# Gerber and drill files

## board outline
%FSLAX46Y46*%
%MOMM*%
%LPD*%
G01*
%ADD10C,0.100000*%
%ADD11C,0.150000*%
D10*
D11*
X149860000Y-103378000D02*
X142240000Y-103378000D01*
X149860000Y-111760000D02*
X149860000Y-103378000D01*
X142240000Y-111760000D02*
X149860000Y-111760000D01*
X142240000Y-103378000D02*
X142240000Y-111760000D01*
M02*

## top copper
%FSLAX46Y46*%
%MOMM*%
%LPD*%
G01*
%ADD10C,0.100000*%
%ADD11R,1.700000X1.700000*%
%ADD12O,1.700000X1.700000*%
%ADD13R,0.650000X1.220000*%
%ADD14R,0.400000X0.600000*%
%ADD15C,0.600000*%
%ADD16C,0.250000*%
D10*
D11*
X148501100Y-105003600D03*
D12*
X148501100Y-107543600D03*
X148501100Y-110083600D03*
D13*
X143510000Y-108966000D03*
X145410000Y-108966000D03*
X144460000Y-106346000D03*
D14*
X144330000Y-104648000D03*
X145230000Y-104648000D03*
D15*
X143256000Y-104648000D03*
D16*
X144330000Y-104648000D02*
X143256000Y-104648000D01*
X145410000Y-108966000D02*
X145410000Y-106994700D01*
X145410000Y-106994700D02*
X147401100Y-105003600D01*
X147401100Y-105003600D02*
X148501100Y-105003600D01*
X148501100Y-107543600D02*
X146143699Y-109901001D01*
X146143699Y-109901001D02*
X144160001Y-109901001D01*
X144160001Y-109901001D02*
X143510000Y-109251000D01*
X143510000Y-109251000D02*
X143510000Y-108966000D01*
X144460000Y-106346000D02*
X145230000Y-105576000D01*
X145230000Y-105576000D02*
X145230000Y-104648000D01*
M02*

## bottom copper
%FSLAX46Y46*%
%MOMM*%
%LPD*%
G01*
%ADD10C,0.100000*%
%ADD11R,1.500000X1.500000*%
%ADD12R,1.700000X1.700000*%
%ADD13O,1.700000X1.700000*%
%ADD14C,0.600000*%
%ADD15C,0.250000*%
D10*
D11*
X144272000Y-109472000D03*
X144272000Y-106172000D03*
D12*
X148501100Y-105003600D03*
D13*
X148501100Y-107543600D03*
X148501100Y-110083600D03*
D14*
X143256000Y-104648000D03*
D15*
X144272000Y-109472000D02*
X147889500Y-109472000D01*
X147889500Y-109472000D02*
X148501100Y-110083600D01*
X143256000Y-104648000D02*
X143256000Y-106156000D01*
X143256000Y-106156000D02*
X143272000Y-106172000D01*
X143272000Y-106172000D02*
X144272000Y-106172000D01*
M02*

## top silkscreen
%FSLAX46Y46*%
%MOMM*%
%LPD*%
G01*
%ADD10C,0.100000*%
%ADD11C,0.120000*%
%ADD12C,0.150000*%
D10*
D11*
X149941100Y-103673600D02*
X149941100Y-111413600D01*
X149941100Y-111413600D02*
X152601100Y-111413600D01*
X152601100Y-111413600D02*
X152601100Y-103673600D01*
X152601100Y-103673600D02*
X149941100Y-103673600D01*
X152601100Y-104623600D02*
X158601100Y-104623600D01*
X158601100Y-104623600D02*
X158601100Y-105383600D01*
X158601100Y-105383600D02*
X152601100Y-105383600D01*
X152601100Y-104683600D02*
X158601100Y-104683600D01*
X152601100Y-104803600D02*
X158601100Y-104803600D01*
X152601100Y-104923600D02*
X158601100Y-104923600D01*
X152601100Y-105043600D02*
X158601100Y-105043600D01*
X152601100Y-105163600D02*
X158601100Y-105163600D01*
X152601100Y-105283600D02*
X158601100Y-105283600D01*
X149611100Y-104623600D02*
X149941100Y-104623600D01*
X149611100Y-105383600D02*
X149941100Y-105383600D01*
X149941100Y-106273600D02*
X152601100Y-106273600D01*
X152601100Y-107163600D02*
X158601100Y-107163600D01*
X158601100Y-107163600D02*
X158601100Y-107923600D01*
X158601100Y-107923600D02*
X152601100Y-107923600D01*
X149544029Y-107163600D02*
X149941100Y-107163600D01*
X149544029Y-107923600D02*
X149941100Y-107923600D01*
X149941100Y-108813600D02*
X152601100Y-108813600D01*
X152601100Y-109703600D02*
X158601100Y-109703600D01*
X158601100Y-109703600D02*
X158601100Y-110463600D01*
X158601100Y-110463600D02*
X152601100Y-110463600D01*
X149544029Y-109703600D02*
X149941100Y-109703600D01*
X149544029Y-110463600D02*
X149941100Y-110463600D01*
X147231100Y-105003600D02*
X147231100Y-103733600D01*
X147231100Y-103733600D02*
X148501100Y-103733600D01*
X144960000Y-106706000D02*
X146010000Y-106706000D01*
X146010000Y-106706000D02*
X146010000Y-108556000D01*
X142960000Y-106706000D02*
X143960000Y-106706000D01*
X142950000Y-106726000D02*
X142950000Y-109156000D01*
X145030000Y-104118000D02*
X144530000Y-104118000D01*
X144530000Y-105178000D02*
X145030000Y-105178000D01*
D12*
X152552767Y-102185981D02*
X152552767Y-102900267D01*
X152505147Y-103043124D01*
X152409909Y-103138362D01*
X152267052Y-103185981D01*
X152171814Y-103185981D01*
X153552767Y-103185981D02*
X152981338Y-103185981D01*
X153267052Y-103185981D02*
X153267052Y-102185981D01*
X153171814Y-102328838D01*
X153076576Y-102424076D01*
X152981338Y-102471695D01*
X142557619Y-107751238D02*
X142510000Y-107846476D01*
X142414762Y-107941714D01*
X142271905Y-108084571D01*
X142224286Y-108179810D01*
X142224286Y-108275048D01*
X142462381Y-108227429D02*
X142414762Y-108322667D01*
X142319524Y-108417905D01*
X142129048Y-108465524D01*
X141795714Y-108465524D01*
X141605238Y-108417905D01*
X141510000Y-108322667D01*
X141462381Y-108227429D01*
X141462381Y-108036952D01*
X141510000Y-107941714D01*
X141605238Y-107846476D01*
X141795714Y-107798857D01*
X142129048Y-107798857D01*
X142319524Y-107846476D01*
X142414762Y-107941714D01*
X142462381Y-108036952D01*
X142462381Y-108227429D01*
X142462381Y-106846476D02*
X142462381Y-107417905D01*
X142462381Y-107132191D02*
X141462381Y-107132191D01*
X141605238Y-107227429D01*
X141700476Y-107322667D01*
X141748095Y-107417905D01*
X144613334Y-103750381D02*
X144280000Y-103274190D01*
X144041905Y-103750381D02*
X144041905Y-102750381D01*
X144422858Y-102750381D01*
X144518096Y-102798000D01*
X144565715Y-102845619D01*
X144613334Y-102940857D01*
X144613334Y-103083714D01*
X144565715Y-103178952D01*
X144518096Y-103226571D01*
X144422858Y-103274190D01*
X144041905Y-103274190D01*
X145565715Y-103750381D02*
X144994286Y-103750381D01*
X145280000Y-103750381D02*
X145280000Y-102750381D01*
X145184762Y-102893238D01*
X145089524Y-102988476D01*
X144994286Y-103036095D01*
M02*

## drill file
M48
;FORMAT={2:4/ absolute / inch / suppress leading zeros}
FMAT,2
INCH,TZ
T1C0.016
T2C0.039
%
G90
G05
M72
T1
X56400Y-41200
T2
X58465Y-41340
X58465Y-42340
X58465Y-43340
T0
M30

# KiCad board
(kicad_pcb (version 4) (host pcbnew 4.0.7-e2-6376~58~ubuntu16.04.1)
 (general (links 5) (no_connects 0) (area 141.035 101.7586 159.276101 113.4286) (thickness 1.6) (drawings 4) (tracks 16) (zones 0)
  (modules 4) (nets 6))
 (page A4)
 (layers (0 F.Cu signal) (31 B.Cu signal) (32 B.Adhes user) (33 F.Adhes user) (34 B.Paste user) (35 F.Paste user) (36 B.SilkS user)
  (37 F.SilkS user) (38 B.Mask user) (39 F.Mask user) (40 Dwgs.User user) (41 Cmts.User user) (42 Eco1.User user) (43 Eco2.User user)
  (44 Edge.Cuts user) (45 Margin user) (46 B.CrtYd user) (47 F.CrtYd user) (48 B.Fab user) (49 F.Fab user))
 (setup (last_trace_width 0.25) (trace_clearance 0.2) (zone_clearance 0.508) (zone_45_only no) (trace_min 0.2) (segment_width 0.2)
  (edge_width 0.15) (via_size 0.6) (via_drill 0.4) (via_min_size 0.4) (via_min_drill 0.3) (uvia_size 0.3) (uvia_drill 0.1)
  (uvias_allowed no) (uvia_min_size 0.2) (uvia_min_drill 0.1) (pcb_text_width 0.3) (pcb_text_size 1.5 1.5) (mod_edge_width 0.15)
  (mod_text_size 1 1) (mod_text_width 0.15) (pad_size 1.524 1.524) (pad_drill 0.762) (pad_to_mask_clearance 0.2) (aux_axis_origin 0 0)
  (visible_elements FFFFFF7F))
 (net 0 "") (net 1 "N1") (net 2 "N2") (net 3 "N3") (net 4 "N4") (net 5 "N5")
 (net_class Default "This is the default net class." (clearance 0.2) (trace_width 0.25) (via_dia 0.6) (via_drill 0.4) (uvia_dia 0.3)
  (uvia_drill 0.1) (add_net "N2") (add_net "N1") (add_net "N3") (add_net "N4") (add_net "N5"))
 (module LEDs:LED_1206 (layer B.Cu) (at 144.272 107.822 270)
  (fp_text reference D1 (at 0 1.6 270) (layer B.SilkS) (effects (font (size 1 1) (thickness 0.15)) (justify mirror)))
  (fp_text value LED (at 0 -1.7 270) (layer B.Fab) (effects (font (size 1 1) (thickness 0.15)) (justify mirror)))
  (pad 2 smd rect (at 1.65 0 90) (size 1.5 1.5) (layers B.Cu B.Paste B.Mask) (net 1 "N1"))
  (pad 1 smd rect (at -1.65 0 90) (size 1.5 1.5) (layers B.Cu B.Paste B.Mask) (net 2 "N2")))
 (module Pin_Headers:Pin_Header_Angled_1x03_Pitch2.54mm (layer F.Cu) (at 148.5011 105.0036)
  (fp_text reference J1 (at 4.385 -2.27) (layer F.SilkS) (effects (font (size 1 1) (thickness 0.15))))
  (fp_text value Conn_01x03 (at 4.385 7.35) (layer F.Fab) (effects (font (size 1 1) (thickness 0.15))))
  (fp_line (start 1.44 -1.33) (end 1.44 6.41) (layer F.SilkS) (width 0.12))
  (fp_line (start 1.44 6.41) (end 4.1 6.41) (layer F.SilkS) (width 0.12))
  (fp_line (start 4.1 6.41) (end 4.1 -1.33) (layer F.SilkS) (width 0.12))
  (fp_line (start 4.1 -1.33) (end 1.44 -1.33) (layer F.SilkS) (width 0.12))
  (fp_line (start 4.1 -0.38) (end 10.1 -0.38) (layer F.SilkS) (width 0.12))
  (fp_line (start 10.1 -0.38) (end 10.1 0.38) (layer F.SilkS) (width 0.12))
  (fp_line (start 10.1 0.38) (end 4.1 0.38) (layer F.SilkS) (width 0.12))
  (fp_line (start 4.1 -0.32) (end 10.1 -0.32) (layer F.SilkS) (width 0.12))
  (fp_line (start 4.1 -0.2) (end 10.1 -0.2) (layer F.SilkS) (width 0.12))
  (fp_line (start 4.1 -0.08) (end 10.1 -0.08) (layer F.SilkS) (width 0.12))
  (fp_line (start 4.1 0.04) (end 10.1 0.04) (layer F.SilkS) (width 0.12))
  (fp_line (start 4.1 0.16) (end 10.1 0.16) (layer F.SilkS) (width 0.12))
  (fp_line (start 4.1 0.28) (end 10.1 0.28) (layer F.SilkS) (width 0.12))
  (fp_line (start 1.11 -0.38) (end 1.44 -0.38) (layer F.SilkS) (width 0.12))
  (fp_line (start 1.11 0.38) (end 1.44 0.38) (layer F.SilkS) (width 0.12))
  (fp_line (start 1.44 1.27) (end 4.1 1.27) (layer F.SilkS) (width 0.12))
  (fp_line (start 4.1 2.16) (end 10.1 2.16) (layer F.SilkS) (width 0.12))
  (fp_line (start 10.1 2.16) (end 10.1 2.92) (layer F.SilkS) (width 0.12))
  (fp_line (start 10.1 2.92) (end 4.1 2.92) (layer F.SilkS) (width 0.12))
  (fp_line (start 1.042929 2.16) (end 1.44 2.16) (layer F.SilkS) (width 0.12))
  (fp_line (start 1.042929 2.92) (end 1.44 2.92) (layer F.SilkS) (width 0.12))
  (fp_line (start 1.44 3.81) (end 4.1 3.81) (layer F.SilkS) (width 0.12))
  (fp_line (start 4.1 4.7) (end 10.1 4.7) (layer F.SilkS) (width 0.12))
  (fp_line (start 10.1 4.7) (end 10.1 5.46) (layer F.SilkS) (width 0.12))
  (fp_line (start 10.1 5.46) (end 4.1 5.46) (layer F.SilkS) (width 0.12))
  (fp_line (start 1.042929 4.7) (end 1.44 4.7) (layer F.SilkS) (width 0.12))
  (fp_line (start 1.042929 5.46) (end 1.44 5.46) (layer F.SilkS) (width 0.12))
  (fp_line (start -1.27 0) (end -1.27 -1.27) (layer F.SilkS) (width 0.12))
  (fp_line (start -1.27 -1.27) (end 0 -1.27) (layer F.SilkS) (width 0.12))
  (pad 1 thru_hole rect (at 0 0) (size 1.7 1.7) (drill 1) (layers *.Cu *.Mask) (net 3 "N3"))
  (pad 2 thru_hole oval (at 0 2.54) (size 1.7 1.7) (drill 1) (layers *.Cu *.Mask) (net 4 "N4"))
  (pad 3 thru_hole oval (at 0 5.08) (size 1.7 1.7) (drill 1) (layers *.Cu *.Mask) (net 1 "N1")))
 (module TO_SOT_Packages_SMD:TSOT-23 (layer F.Cu) (at 144.46 107.656 90)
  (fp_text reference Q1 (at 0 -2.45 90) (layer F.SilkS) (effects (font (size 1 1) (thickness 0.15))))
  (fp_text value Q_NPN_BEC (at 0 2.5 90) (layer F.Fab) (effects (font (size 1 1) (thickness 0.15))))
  (fp_line (start 0.95 0.5) (end 0.95 1.55) (layer F.SilkS) (width 0.12))
  (fp_line (start 0.95 1.55) (end -0.9 1.55) (layer F.SilkS) (width 0.12))
  (fp_line (start 0.95 -1.5) (end 0.95 -0.5) (layer F.SilkS) (width 0.12))
  (fp_line (start 0.93 -1.51) (end -1.5 -1.51) (layer F.SilkS) (width 0.12))
  (pad 1 smd rect (at -1.31 -0.95 90) (size 1.22 0.65) (layers F.Cu F.Paste F.Mask) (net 4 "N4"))
  (pad 2 smd rect (at -1.31 0.95 90) (size 1.22 0.65) (layers F.Cu F.Paste F.Mask) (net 3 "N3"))
  (pad 3 smd rect (at 1.31 0 90) (size 1.22 0.65) (layers F.Cu F.Paste F.Mask) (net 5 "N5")))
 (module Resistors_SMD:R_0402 (layer F.Cu) (at 144.78 104.648)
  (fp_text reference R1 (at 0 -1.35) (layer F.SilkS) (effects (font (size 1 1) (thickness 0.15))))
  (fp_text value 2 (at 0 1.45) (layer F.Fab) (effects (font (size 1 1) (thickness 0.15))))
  (fp_line (start 0.25 -0.53) (end -0.25 -0.53) (layer F.SilkS) (width 0.12))
  (fp_line (start -0.25 0.53) (end 0.25 0.53) (layer F.SilkS) (width 0.12))
  (pad 1 smd rect (at -0.45 0) (size 0.4 0.6) (layers F.Cu F.Paste F.Mask) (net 2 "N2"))
  (pad 2 smd rect (at 0.45 0) (size 0.4 0.6) (layers F.Cu F.Paste F.Mask) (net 5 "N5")))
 (gr_line (start 149.86 103.378) (end 142.24 103.378) (layer Edge.Cuts) (width 0.15))
 (gr_line (start 149.86 111.76) (end 149.86 103.378) (layer Edge.Cuts) (width 0.15))
 (gr_line (start 142.24 111.76) (end 149.86 111.76) (layer Edge.Cuts) (width 0.15))
 (gr_line (start 142.24 103.378) (end 142.24 111.76) (layer Edge.Cuts) (width 0.15))
 (segment (start 144.272 109.472) (end 147.8895 109.472) (width 0.25) (layer B.Cu) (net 1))
 (segment (start 147.8895 109.472) (end 148.5011 110.0836) (width 0.25) (layer B.Cu) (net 1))
 (segment (start 143.256 104.648) (end 143.256 106.156) (width 0.25) (layer B.Cu) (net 2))
 (segment (start 143.256 106.156) (end 143.272 106.172) (width 0.25) (layer B.Cu) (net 2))
 (segment (start 143.272 106.172) (end 144.272 106.172) (width 0.25) (layer B.Cu) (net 2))
 (segment (start 144.33 104.648) (end 143.256 104.648) (width 0.25) (layer F.Cu) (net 2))
 (via (at 143.256 104.648) (size 0.6) (drill 0.4) (layers F.Cu B.Cu) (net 2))
 (segment (start 145.41 108.966) (end 145.41 106.9947) (width 0.25) (layer F.Cu) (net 3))
 (segment (start 145.41 106.9947) (end 147.4011 105.0036) (width 0.25) (layer F.Cu) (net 3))
 (segment (start 147.4011 105.0036) (end 148.5011 105.0036) (width 0.25) (layer F.Cu) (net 3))
 (segment (start 148.5011 107.5436) (end 146.143699 109.901001) (width 0.25) (layer F.Cu) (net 4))
 (segment (start 146.143699 109.901001) (end 144.160001 109.901001) (width 0.25) (layer F.Cu) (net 4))
 (segment (start 144.160001 109.901001) (end 143.51 109.251) (width 0.25) (layer F.Cu) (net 4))
 (segment (start 143.51 109.251) (end 143.51 108.966) (width 0.25) (layer F.Cu) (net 4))
 (segment (start 144.46 106.346) (end 145.23 105.576) (width 0.25) (layer F.Cu) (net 5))
 (segment (start 145.23 105.576) (end 145.23 104.648) (width 0.25) (layer F.Cu) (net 5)))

